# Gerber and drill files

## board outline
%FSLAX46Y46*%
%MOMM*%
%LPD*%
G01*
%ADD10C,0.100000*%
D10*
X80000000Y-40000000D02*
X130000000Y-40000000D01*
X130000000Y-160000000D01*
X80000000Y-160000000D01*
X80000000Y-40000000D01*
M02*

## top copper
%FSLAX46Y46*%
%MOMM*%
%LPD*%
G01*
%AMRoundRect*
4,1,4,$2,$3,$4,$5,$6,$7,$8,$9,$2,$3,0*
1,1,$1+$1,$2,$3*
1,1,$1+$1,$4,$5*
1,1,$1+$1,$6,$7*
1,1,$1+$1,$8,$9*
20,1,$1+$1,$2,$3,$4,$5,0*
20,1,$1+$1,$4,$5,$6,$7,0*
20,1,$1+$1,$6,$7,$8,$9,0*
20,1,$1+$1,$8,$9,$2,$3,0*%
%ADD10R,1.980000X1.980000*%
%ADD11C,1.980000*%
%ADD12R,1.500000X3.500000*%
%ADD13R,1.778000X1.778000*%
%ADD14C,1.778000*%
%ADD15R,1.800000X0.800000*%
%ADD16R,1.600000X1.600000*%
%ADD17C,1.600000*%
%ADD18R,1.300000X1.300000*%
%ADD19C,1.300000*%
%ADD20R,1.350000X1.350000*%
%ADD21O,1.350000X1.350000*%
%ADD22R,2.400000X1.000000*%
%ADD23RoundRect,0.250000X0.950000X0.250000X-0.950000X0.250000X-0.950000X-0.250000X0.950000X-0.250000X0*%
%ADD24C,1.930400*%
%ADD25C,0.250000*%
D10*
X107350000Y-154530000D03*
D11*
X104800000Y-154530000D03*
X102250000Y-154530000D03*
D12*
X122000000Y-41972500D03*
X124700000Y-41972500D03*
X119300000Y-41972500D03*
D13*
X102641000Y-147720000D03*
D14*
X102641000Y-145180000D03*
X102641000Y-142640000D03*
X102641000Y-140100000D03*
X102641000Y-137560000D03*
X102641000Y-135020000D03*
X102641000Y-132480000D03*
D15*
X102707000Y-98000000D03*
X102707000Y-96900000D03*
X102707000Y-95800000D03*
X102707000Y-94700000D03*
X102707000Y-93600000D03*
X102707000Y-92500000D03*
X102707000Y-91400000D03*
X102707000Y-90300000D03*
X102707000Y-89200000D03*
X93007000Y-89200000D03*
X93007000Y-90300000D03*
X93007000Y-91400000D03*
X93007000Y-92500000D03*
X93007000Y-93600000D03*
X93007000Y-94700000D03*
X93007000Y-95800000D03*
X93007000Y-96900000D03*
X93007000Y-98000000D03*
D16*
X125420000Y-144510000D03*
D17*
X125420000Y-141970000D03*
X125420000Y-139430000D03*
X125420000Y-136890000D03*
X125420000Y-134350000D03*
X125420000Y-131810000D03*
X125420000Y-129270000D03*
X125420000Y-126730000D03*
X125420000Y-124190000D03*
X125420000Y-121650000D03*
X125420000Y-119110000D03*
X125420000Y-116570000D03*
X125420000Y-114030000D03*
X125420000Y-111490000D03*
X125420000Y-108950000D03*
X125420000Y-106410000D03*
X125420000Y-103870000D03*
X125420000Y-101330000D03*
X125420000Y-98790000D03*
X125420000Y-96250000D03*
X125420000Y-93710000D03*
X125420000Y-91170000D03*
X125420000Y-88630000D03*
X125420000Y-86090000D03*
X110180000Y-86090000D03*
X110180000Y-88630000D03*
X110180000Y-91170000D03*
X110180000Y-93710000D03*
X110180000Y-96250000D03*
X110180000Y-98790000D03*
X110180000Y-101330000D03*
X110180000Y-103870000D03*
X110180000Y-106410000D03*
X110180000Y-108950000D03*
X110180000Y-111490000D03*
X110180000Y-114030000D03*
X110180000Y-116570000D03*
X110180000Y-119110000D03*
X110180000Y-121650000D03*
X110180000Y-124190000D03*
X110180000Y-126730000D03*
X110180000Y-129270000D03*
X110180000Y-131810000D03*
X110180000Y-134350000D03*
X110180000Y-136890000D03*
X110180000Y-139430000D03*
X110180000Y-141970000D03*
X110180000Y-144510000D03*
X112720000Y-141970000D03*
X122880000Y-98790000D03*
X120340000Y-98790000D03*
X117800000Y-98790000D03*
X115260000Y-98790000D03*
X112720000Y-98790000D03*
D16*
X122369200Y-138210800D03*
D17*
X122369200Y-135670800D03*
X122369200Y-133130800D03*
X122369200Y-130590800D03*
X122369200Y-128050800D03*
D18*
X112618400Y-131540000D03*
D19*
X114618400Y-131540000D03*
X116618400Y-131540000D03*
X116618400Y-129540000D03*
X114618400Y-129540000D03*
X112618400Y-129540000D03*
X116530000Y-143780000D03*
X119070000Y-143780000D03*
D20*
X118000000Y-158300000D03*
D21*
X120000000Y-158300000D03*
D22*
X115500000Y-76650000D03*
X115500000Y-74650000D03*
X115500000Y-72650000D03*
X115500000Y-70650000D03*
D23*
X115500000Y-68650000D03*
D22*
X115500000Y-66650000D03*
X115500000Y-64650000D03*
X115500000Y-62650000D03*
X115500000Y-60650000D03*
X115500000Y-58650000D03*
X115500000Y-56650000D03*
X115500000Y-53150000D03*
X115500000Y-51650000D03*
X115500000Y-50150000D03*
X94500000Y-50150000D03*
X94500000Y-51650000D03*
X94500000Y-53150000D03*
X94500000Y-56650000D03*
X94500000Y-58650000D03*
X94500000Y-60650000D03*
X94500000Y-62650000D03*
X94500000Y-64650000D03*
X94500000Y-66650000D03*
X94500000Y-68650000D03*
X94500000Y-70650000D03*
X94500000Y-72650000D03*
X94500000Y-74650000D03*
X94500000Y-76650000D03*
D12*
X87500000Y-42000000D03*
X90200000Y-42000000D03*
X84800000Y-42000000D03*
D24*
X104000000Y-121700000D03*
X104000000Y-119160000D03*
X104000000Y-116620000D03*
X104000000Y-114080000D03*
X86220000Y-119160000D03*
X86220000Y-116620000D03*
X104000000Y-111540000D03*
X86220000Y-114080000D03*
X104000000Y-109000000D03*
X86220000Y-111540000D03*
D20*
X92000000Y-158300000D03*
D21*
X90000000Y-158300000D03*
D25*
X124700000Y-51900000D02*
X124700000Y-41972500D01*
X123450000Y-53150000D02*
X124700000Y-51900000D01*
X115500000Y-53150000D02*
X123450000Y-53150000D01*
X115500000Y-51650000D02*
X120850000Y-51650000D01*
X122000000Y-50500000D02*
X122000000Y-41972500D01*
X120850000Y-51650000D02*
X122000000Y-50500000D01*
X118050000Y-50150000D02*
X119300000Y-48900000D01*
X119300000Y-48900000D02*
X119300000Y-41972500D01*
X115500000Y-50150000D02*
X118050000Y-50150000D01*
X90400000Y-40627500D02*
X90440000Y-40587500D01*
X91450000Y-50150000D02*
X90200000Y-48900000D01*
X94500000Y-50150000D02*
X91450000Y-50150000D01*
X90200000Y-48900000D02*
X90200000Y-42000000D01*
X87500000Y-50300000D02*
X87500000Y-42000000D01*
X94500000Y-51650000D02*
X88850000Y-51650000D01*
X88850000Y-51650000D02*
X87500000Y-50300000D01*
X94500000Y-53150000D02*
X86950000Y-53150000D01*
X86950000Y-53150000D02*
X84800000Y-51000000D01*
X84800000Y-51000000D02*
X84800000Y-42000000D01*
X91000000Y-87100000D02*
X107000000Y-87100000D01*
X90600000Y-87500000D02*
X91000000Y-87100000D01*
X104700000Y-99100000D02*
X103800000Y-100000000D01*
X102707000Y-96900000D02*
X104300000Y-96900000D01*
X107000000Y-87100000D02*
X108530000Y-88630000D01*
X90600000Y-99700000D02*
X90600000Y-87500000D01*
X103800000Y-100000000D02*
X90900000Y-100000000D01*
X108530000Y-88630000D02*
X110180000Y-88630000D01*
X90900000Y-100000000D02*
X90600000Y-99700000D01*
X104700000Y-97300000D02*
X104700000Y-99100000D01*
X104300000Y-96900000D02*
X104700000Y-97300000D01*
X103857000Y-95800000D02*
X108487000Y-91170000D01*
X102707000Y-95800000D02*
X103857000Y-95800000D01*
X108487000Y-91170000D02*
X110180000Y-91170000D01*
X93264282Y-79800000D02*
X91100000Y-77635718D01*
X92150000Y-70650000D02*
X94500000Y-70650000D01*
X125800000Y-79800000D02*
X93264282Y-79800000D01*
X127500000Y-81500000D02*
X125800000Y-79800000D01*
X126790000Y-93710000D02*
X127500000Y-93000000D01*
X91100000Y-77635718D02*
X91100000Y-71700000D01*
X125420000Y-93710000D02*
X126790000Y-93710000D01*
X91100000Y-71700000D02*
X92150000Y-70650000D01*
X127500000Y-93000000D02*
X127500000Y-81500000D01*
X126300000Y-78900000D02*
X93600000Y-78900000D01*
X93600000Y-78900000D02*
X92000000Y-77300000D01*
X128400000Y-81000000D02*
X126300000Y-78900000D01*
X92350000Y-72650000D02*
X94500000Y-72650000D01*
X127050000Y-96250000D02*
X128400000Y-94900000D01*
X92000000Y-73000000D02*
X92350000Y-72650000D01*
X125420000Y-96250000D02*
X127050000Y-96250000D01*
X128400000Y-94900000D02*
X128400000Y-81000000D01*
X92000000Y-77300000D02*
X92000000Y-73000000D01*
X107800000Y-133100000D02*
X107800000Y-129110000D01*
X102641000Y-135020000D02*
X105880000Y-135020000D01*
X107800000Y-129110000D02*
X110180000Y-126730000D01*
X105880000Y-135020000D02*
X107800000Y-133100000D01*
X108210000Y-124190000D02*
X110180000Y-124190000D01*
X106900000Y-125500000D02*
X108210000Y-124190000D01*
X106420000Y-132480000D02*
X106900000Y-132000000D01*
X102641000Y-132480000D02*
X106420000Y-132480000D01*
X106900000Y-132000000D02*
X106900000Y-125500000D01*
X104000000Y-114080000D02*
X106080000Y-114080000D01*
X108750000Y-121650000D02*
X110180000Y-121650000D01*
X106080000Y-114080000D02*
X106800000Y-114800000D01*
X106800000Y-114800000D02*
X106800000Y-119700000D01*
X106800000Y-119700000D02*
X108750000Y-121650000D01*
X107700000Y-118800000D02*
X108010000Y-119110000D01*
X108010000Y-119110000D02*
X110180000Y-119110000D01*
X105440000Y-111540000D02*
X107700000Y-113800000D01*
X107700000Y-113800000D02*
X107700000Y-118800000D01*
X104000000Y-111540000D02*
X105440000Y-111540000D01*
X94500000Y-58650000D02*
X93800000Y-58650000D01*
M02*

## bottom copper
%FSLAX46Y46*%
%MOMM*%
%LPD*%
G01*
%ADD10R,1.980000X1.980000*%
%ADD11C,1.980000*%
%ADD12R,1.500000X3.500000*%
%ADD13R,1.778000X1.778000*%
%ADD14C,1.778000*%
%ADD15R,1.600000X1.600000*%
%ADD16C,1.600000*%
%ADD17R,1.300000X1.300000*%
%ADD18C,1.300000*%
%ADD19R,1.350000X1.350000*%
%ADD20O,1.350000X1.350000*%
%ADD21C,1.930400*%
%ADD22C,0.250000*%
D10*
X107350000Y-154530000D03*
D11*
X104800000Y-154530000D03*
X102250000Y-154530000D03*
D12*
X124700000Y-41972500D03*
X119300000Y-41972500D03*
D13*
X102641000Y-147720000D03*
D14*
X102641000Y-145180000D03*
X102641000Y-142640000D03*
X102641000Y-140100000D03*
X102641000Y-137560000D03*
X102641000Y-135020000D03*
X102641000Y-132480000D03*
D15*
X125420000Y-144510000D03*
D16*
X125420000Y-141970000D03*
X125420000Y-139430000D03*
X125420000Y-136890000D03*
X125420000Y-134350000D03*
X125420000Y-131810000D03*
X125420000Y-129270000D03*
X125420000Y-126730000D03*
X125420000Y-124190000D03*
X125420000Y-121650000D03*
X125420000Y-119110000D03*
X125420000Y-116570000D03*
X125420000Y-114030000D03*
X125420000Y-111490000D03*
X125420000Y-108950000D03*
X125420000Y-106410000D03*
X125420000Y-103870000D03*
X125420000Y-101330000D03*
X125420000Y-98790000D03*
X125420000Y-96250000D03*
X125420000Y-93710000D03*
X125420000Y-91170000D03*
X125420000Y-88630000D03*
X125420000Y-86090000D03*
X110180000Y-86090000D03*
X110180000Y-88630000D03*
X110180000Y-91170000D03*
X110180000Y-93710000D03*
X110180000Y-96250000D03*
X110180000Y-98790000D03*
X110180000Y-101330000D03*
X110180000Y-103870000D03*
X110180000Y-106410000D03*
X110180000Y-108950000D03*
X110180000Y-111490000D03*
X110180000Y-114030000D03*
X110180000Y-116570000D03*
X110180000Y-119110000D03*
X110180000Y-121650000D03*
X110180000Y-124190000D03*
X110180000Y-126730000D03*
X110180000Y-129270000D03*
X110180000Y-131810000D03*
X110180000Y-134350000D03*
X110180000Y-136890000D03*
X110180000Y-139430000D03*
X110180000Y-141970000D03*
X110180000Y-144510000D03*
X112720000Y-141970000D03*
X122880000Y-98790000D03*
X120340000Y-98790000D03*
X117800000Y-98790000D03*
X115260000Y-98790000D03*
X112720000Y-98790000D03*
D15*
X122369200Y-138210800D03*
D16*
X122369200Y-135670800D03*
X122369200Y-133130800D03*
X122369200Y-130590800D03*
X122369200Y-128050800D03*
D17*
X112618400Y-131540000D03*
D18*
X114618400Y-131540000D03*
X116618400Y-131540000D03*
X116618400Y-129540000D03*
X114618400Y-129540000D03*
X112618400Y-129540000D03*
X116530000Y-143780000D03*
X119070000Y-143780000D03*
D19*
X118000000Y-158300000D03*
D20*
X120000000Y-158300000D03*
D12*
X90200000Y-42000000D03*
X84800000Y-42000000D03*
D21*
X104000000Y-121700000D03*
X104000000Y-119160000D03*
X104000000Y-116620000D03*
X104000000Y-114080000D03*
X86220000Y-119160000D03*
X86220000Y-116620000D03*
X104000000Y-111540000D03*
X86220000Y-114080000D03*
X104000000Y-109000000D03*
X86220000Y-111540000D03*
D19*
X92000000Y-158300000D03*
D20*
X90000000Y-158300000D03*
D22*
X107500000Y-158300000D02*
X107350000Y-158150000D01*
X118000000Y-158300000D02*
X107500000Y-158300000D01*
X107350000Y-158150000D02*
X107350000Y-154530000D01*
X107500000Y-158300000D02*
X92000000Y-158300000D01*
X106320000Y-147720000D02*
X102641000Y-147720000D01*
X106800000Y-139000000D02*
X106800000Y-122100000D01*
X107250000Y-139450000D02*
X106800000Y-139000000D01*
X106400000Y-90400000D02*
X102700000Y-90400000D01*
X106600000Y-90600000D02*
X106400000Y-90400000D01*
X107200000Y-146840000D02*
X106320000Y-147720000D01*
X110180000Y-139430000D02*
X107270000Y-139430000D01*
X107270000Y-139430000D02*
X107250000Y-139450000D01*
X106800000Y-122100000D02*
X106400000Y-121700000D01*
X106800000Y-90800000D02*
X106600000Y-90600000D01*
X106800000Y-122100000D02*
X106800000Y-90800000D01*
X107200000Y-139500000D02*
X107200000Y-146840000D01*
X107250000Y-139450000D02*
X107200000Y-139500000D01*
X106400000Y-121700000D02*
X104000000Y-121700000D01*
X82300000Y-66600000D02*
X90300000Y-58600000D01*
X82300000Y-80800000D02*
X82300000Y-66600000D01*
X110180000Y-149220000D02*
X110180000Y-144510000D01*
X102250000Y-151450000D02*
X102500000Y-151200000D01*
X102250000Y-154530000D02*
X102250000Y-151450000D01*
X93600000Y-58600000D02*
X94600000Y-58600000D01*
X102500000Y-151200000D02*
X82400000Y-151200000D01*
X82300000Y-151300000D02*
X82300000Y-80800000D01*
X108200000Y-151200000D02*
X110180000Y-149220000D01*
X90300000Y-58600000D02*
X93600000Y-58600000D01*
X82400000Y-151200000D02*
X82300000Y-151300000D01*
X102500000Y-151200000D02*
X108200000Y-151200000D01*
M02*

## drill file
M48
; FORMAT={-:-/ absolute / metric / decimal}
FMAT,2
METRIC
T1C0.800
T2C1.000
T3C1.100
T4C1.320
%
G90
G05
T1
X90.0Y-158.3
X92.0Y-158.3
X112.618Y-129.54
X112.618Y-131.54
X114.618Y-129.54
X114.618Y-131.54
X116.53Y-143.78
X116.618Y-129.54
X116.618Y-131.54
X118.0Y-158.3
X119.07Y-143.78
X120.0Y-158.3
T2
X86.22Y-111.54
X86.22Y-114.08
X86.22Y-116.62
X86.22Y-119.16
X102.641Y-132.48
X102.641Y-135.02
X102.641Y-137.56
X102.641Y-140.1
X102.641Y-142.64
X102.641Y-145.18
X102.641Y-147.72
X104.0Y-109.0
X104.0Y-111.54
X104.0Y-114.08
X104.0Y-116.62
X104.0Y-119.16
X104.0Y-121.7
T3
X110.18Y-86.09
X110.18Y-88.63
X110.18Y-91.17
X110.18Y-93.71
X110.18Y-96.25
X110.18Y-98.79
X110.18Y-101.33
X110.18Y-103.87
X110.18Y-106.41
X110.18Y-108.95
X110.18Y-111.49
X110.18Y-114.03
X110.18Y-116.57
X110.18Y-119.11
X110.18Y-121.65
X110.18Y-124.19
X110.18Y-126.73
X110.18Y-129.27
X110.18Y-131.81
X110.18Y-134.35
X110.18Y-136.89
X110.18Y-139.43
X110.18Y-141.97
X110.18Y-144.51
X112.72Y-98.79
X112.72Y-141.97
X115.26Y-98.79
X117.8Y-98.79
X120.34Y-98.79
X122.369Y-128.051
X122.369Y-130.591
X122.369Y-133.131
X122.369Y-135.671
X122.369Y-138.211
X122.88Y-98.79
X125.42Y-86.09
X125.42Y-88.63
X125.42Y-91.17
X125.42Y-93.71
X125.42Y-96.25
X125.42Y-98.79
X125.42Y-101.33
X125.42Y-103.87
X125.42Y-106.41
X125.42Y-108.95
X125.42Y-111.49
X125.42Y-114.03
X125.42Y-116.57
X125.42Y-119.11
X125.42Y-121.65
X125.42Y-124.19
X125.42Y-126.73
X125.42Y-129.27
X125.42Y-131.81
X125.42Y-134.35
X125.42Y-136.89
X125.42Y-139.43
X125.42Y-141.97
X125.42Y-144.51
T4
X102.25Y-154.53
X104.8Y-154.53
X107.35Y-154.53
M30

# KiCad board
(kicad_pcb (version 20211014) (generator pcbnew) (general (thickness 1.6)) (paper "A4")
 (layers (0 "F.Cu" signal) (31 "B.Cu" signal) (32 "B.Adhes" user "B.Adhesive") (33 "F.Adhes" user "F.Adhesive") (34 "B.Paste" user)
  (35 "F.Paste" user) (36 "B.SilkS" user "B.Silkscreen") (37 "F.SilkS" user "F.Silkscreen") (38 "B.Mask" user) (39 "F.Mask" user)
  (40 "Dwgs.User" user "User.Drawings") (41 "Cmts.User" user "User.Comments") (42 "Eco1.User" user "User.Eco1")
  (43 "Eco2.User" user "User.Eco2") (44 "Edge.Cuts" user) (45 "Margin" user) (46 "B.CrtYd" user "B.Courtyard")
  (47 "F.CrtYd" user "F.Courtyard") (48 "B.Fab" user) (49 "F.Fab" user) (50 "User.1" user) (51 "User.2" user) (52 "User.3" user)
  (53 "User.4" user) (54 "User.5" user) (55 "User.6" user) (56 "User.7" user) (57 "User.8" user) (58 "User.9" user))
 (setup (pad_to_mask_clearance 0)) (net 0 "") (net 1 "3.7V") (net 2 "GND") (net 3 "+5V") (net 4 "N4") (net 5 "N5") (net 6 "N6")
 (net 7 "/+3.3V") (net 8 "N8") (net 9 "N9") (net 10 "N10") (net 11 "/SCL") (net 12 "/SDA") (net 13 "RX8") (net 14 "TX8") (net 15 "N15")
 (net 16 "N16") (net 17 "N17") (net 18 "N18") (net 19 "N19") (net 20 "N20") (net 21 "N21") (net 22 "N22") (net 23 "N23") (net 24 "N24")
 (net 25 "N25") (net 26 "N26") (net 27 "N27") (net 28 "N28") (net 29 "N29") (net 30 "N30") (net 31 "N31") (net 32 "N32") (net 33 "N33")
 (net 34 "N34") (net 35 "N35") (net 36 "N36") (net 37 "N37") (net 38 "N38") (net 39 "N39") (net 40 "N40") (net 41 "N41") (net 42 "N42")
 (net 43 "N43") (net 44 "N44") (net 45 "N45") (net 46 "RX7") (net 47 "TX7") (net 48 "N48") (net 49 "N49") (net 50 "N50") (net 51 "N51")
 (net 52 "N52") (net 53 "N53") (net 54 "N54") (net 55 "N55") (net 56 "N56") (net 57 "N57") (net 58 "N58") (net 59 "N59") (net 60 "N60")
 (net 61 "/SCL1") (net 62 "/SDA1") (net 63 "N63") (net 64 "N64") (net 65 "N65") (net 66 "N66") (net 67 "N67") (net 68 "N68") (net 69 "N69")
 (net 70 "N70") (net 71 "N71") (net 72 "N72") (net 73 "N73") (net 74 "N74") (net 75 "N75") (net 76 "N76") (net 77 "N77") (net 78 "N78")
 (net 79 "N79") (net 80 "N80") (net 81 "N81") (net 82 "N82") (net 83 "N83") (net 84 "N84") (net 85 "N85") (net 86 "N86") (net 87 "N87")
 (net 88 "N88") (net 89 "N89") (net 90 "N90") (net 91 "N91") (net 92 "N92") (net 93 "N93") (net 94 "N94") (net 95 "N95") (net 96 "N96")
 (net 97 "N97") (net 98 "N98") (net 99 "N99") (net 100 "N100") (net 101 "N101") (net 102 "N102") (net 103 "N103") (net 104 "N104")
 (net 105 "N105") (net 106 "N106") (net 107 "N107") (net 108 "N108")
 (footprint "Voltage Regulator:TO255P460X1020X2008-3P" (layer "F.Cu") (at 107.35 154.53 180)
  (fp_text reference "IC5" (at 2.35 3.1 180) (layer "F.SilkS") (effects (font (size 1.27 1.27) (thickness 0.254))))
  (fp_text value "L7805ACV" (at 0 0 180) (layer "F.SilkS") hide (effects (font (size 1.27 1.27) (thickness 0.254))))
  (pad "1" thru_hole rect (at 0 0 180) (size 1.98 1.98) (drill 1.32) (layers *.Cu *.Mask) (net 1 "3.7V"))
  (pad "2" thru_hole circle (at 2.55 0 180) (size 1.98 1.98) (drill 1.32) (layers *.Cu *.Mask) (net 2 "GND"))
  (pad "3" thru_hole circle (at 5.1 0 180) (size 1.98 1.98) (drill 1.32) (layers *.Cu *.Mask) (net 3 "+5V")))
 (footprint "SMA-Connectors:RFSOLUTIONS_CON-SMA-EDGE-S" (layer "F.Cu") (at 122 41.9725 -90)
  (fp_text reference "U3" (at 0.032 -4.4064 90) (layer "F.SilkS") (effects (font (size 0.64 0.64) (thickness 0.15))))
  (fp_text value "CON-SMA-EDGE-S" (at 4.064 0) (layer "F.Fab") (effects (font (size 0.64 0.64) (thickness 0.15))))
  (pad "1" smd rect (at 0 0 270) (size 3.5 1.5) (layers "F.Cu" "F.Paste" "F.Mask") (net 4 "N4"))
  (pad "G1" smd rect (at 0 -2.7 270) (size 3.5 1.5) (layers "F.Cu" "F.Paste" "F.Mask") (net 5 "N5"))
  (pad "G2" smd rect (at 0 2.7 270) (size 3.5 1.5) (layers "F.Cu" "F.Paste" "F.Mask") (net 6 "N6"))
  (pad "G3" smd rect (at 0 -2.7 270) (size 3.5 1.5) (layers "B.Cu" "B.Paste" "B.Mask"))
  (pad "G4" smd rect (at 0 2.7 270) (size 3.5 1.5) (layers "B.Cu" "B.Paste" "B.Mask")))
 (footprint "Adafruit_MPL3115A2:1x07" (layer "F.Cu") (at 100.101 140.1 90)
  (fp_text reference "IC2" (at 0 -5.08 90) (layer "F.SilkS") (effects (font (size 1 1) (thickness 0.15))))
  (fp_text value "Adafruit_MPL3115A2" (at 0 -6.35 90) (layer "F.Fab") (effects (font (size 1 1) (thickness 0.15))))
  (pad "1" thru_hole rect (at -7.62 2.54 180) (size 1.778 1.778) (drill 1) (layers *.Cu *.Mask) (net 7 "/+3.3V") (solder_mask_margin 0.0508))
  (pad "2" thru_hole circle (at -5.08 2.54 90) (size 1.778 1.778) (drill 1) (layers *.Cu *.Mask) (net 2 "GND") (solder_mask_margin 0.0508))
  (pad "3" thru_hole circle (at -2.54 2.54 90) (size 1.778 1.778) (drill 1) (layers *.Cu *.Mask) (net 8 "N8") (solder_mask_margin 0.0508))
  (pad "4" thru_hole circle (at 0 2.54 90) (size 1.778 1.778) (drill 1) (layers *.Cu *.Mask) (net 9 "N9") (solder_mask_margin 0.0508))
  (pad "5" thru_hole circle (at 2.54 2.54 90) (size 1.778 1.778) (drill 1) (layers *.Cu *.Mask) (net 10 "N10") (solder_mask_margin 0.0508))
  (pad "6" thru_hole circle (at 5.08 2.54 90) (size 1.778 1.778) (drill 1) (layers *.Cu *.Mask) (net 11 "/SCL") (solder_mask_margin 0.0508))
  (pad "7" thru_hole circle (at 7.62 2.54 90) (size 1.778 1.778) (drill 1) (layers *.Cu *.Mask) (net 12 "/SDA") (solder_mask_margin 0.0508)))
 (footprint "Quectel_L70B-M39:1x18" (layer "F.Cu") (at 97.857 93.6 180)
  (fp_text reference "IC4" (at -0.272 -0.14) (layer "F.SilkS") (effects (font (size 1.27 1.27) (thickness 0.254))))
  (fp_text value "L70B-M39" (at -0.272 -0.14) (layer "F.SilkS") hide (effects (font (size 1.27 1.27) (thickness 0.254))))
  (pad "1" smd rect (at -4.85 -4.4 270) (size 0.8 1.8) (layers "F.Cu" "F.Paste" "F.Mask") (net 2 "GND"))
  (pad "2" smd rect (at -4.85 -3.3 270) (size 0.8 1.8) (layers "F.Cu" "F.Paste" "F.Mask") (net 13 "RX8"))
  (pad "3" smd rect (at -4.85 -2.2 270) (size 0.8 1.8) (layers "F.Cu" "F.Paste" "F.Mask") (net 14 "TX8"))
  (pad "4" smd rect (at -4.85 -1.1 270) (size 0.8 1.8) (layers "F.Cu" "F.Paste" "F.Mask") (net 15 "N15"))
  (pad "5" smd rect (at -4.85 0 270) (size 0.8 1.8) (layers "F.Cu" "F.Paste" "F.Mask") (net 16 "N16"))
  (pad "6" smd rect (at -4.85 1.1 270) (size 0.8 1.8) (layers "F.Cu" "F.Paste" "F.Mask") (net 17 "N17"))
  (pad "7" smd rect (at -4.85 2.2 270) (size 0.8 1.8) (layers "F.Cu" "F.Paste" "F.Mask") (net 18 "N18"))
  (pad "8" smd rect (at -4.85 3.3 270) (size 0.8 1.8) (layers "F.Cu" "F.Paste" "F.Mask") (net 7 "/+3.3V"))
  (pad "9" smd rect (at -4.85 4.4 270) (size 0.8 1.8) (layers "F.Cu" "F.Paste" "F.Mask") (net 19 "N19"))
  (pad "10" smd rect (at 4.85 4.4 270) (size 0.8 1.8) (layers "F.Cu" "F.Paste" "F.Mask") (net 2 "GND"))
  (pad "11" smd rect (at 4.85 3.3 270) (size 0.8 1.8) (layers "F.Cu" "F.Paste" "F.Mask") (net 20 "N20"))
  (pad "12" smd rect (at 4.85 2.2 270) (size 0.8 1.8) (layers "F.Cu" "F.Paste" "F.Mask") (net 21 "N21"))
  (pad "13" smd rect (at 4.85 1.1 270) (size 0.8 1.8) (layers "F.Cu" "F.Paste" "F.Mask") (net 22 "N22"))
  (pad "14" smd rect (at 4.85 0 270) (size 0.8 1.8) (layers "F.Cu" "F.Paste" "F.Mask") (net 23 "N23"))
  (pad "15" smd rect (at 4.85 -1.1 270) (size 0.8 1.8) (layers "F.Cu" "F.Paste" "F.Mask") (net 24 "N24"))
  (pad "16" smd rect (at 4.85 -2.2 270) (size 0.8 1.8) (layers "F.Cu" "F.Paste" "F.Mask") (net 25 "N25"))
  (pad "17" smd rect (at 4.85 -3.3 270) (size 0.8 1.8) (layers "F.Cu" "F.Paste" "F.Mask") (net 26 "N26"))
  (pad "18" smd rect (at 4.85 -4.4 270) (size 0.8 1.8) (layers "F.Cu" "F.Paste" "F.Mask") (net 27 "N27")))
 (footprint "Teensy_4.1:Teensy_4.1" (layer "F.Cu") (at 117.8 115.3 90)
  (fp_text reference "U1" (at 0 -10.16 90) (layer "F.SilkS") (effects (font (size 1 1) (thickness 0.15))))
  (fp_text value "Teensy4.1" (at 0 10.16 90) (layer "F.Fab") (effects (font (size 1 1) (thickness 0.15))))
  (pad "1" thru_hole rect (at -29.21 7.62 90) (size 1.6 1.6) (drill 1.1) (layers *.Cu *.Mask) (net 2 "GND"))
  (pad "2" thru_hole circle (at -26.67 7.62 90) (size 1.6 1.6) (drill 1.1) (layers *.Cu *.Mask) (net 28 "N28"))
  (pad "3" thru_hole circle (at -24.13 7.62 90) (size 1.6 1.6) (drill 1.1) (layers *.Cu *.Mask) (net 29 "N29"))
  (pad "4" thru_hole circle (at -21.59 7.62 90) (size 1.6 1.6) (drill 1.1) (layers *.Cu *.Mask) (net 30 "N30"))
  (pad "5" thru_hole circle (at -19.05 7.62 90) (size 1.6 1.6) (drill 1.1) (layers *.Cu *.Mask) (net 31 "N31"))
  (pad "6" thru_hole circle (at -16.51 7.62 90) (size 1.6 1.6) (drill 1.1) (layers *.Cu *.Mask) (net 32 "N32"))
  (pad "7" thru_hole circle (at -13.97 7.62 90) (size 1.6 1.6) (drill 1.1) (layers *.Cu *.Mask) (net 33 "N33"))
  (pad "8" thru_hole circle (at -11.43 7.62 90) (size 1.6 1.6) (drill 1.1) (layers *.Cu *.Mask) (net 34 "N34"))
  (pad "9" thru_hole circle (at -8.89 7.62 90) (size 1.6 1.6) (drill 1.1) (layers *.Cu *.Mask) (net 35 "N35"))
  (pad "10" thru_hole circle (at -6.35 7.62 90) (size 1.6 1.6) (drill 1.1) (layers *.Cu *.Mask) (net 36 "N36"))
  (pad "11" thru_hole circle (at -3.81 7.62 90) (size 1.6 1.6) (drill 1.1) (layers *.Cu *.Mask) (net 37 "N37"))
  (pad "12" thru_hole circle (at -1.27 7.62 90) (size 1.6 1.6) (drill 1.1) (layers *.Cu *.Mask) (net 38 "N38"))
  (pad "13" thru_hole circle (at 1.27 7.62 90) (size 1.6 1.6) (drill 1.1) (layers *.Cu *.Mask) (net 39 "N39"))
  (pad "14" thru_hole circle (at 3.81 7.62 90) (size 1.6 1.6) (drill 1.1) (layers *.Cu *.Mask) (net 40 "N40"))
  (pad "15" thru_hole circle (at 6.35 7.62 90) (size 1.6 1.6) (drill 1.1) (layers *.Cu *.Mask) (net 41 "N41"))
  (pad "16" thru_hole circle (at 8.89 7.62 90) (size 1.6 1.6) (drill 1.1) (layers *.Cu *.Mask) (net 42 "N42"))
  (pad "17" thru_hole circle (at 11.43 7.62 90) (size 1.6 1.6) (drill 1.1) (layers *.Cu *.Mask) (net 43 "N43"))
  (pad "18" thru_hole circle (at 13.97 7.62 90) (size 1.6 1.6) (drill 1.1) (layers *.Cu *.Mask) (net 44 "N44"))
  (pad "19" thru_hole circle (at 16.51 7.62 90) (size 1.6 1.6) (drill 1.1) (layers *.Cu *.Mask) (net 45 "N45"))
  (pad "20" thru_hole circle (at 19.05 7.62 90) (size 1.6 1.6) (drill 1.1) (layers *.Cu *.Mask) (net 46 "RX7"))
  (pad "21" thru_hole circle (at 21.59 7.62 90) (size 1.6 1.6) (drill 1.1) (layers *.Cu *.Mask) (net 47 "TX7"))
  (pad "22" thru_hole circle (at 24.13 7.62 90) (size 1.6 1.6) (drill 1.1) (layers *.Cu *.Mask) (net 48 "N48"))
  (pad "23" thru_hole circle (at 26.67 7.62 90) (size 1.6 1.6) (drill 1.1) (layers *.Cu *.Mask) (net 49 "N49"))
  (pad "24" thru_hole circle (at 29.21 7.62 90) (size 1.6 1.6) (drill 1.1) (layers *.Cu *.Mask) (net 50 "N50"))
  (pad "25" thru_hole circle (at 29.21 -7.62 90) (size 1.6 1.6) (drill 1.1) (layers *.Cu *.Mask) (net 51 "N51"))
  (pad "26" thru_hole circle (at 26.67 -7.62 90) (size 1.6 1.6) (drill 1.1) (layers *.Cu *.Mask) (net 13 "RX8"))
  (pad "27" thru_hole circle (at 24.13 -7.62 90) (size 1.6 1.6) (drill 1.1) (layers *.Cu *.Mask) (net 14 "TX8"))
  (pad "28" thru_hole circle (at 21.59 -7.62 90) (size 1.6 1.6) (drill 1.1) (layers *.Cu *.Mask) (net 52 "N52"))
  (pad "29" thru_hole circle (at 19.05 -7.62 90) (size 1.6 1.6) (drill 1.1) (layers *.Cu *.Mask) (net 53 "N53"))
  (pad "30" thru_hole circle (at 16.51 -7.62 90) (size 1.6 1.6) (drill 1.1) (layers *.Cu *.Mask) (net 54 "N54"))
  (pad "31" thru_hole circle (at 13.97 -7.62 90) (size 1.6 1.6) (drill 1.1) (layers *.Cu *.Mask) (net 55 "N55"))
  (pad "32" thru_hole circle (at 11.43 -7.62 90) (size 1.6 1.6) (drill 1.1) (layers *.Cu *.Mask) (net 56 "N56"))
  (pad "33" thru_hole circle (at 8.89 -7.62 90) (size 1.6 1.6) (drill 1.1) (layers *.Cu *.Mask) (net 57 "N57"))
  (pad "34" thru_hole circle (at 6.35 -7.62 90) (size 1.6 1.6) (drill 1.1) (layers *.Cu *.Mask) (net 2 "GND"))
  (pad "35" thru_hole circle (at 3.81 -7.62 90) (size 1.6 1.6) (drill 1.1) (layers *.Cu *.Mask) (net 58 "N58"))
  (pad "36" thru_hole circle (at 1.27 -7.62 90) (size 1.6 1.6) (drill 1.1) (layers *.Cu *.Mask) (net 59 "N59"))
  (pad "37" thru_hole circle (at -1.27 -7.62 90) (size 1.6 1.6) (drill 1.1) (layers *.Cu *.Mask) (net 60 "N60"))
  (pad "38" thru_hole circle (at -3.81 -7.62 90) (size 1.6 1.6) (drill 1.1) (layers *.Cu *.Mask) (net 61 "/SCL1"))
  (pad "39" thru_hole circle (at -6.35 -7.62 90) (size 1.6 1.6) (drill 1.1) (layers *.Cu *.Mask) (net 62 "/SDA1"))
  (pad "40" thru_hole circle (at -8.89 -7.62 90) (size 1.6 1.6) (drill 1.1) (layers *.Cu *.Mask) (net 12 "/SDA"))
  (pad "41" thru_hole circle (at -11.43 -7.62 90) (size 1.6 1.6) (drill 1.1) (layers *.Cu *.Mask) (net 11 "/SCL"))
  (pad "42" thru_hole circle (at -13.97 -7.62 90) (size 1.6 1.6) (drill 1.1) (layers *.Cu *.Mask) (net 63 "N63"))
  (pad "43" thru_hole circle (at -16.51 -7.62 90) (size 1.6 1.6) (drill 1.1) (layers *.Cu *.Mask) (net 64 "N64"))
  (pad "44" thru_hole circle (at -19.05 -7.62 90) (size 1.6 1.6) (drill 1.1) (layers *.Cu *.Mask) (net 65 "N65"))
  (pad "45" thru_hole circle (at -21.59 -7.62 90) (size 1.6 1.6) (drill 1.1) (layers *.Cu *.Mask) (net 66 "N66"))
  (pad "46" thru_hole circle (at -24.13 -7.62 90) (size 1.6 1.6) (drill 1.1) (layers *.Cu *.Mask) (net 7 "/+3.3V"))
  (pad "47" thru_hole circle (at -26.67 -7.62 90) (size 1.6 1.6) (drill 1.1) (layers *.Cu *.Mask) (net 2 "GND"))
  (pad "48" thru_hole circle (at -29.21 -7.62 90) (size 1.6 1.6) (drill 1.1) (layers *.Cu *.Mask) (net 3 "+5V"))
  (pad "49" thru_hole circle (at -26.67 -5.08 90) (size 1.6 1.6) (drill 1.1) (layers *.Cu *.Mask) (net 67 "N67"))
  (pad "50" thru_hole circle (at 16.51 5.08 90) (size 1.6 1.6) (drill 1.1) (layers *.Cu *.Mask) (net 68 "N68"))
  (pad "51" thru_hole circle (at 16.51 2.54 90) (size 1.6 1.6) (drill 1.1) (layers *.Cu *.Mask) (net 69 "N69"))
  (pad "52" thru_hole circle (at 16.51 0 90) (size 1.6 1.6) (drill 1.1) (layers *.Cu *.Mask) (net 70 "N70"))
  (pad "53" thru_hole circle (at 16.51 -2.54 90) (size 1.6 1.6) (drill 1.1) (layers *.Cu *.Mask) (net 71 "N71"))
  (pad "54" thru_hole circle (at 16.51 -5.08 90) (size 1.6 1.6) (drill 1.1) (layers *.Cu *.Mask) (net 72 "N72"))
  (pad "55" thru_hole rect (at -22.9108 4.5692 90) (size 1.6 1.6) (drill 1.1) (layers *.Cu *.Mask) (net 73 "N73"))
  (pad "56" thru_hole circle (at -20.3708 4.5692 90) (size 1.6 1.6) (drill 1.1) (layers *.Cu *.Mask) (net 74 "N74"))
  (pad "57" thru_hole circle (at -17.8308 4.5692 90) (size 1.6 1.6) (drill 1.1) (layers *.Cu *.Mask) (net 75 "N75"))
  (pad "58" thru_hole circle (at -15.2908 4.5692 90) (size 1.6 1.6) (drill 1.1) (layers *.Cu *.Mask) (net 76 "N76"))
  (pad "59" thru_hole circle (at -12.7508 4.5692 90) (size 1.6 1.6) (drill 1.1) (layers *.Cu *.Mask) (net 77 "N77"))
  (pad "60" thru_hole rect (at -16.24 -5.1816 90) (size 1.3 1.3) (drill 0.8) (layers *.Cu *.Mask) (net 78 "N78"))
  (pad "61" thru_hole circle (at -16.24 -3.1816 90) (size 1.3 1.3) (drill 0.8) (layers *.Cu *.Mask) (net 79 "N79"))
  (pad "62" thru_hole circle (at -16.24 -1.1816 90) (size 1.3 1.3) (drill 0.8) (layers *.Cu *.Mask) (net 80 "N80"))
  (pad "63" thru_hole circle (at -14.24 -1.1816 90) (size 1.3 1.3) (drill 0.8) (layers *.Cu *.Mask) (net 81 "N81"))
  (pad "64" thru_hole circle (at -14.24 -3.1816 90) (size 1.3 1.3) (drill 0.8) (layers *.Cu *.Mask) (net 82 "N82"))
  (pad "65" thru_hole circle (at -14.24 -5.1816 90) (size 1.3 1.3) (drill 0.8) (layers *.Cu *.Mask) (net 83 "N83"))
  (pad "66" thru_hole circle (at -28.48 -1.27 90) (size 1.3 1.3) (drill 0.8) (layers *.Cu *.Mask) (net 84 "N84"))
  (pad "67" thru_hole circle (at -28.48 1.27 90) (size 1.3 1.3) (drill 0.8) (layers *.Cu *.Mask) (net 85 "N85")))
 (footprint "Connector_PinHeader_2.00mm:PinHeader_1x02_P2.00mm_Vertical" (layer "F.Cu") (at 118 158.3 90)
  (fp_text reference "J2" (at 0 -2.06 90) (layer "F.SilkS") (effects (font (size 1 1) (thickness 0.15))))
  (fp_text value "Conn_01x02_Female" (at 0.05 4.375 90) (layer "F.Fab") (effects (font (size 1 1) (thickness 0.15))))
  (pad "1" thru_hole rect (at 0 0 90) (size 1.35 1.35) (drill 0.8) (layers *.Cu *.Mask) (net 1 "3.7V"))
  (pad "2" thru_hole oval (at 0 2 90) (size 1.35 1.35) (drill 0.8) (layers *.Cu *.Mask) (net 2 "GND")))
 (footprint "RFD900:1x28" (layer "F.Cu") (at 109.5 66.65 180)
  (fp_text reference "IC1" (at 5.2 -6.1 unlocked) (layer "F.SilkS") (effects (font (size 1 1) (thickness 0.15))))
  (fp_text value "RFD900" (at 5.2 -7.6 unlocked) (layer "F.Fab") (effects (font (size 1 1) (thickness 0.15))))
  (pad "1" smd rect (at -6 -10 180) (size 2.4 1) (layers "F.Cu" "F.Paste" "F.Mask") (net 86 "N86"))
  (pad "2" smd rect (at -6 -8 180) (size 2.4 1) (layers "F.Cu" "F.Paste" "F.Mask") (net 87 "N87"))
  (pad "3" smd rect (at -6 -6 180) (size 2.4 1) (layers "F.Cu" "F.Paste" "F.Mask") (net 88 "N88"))
  (pad "4" smd rect (at -6 -4 180) (size 2.4 1) (layers "F.Cu" "F.Paste" "F.Mask") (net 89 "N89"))
  (pad "5" smd roundrect (at -6 -2 180) (size 2.4 1) (layers "F.Cu" "F.Paste" "F.Mask") (roundrect_rratio 0.25) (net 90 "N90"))
  (pad "6" smd rect (at -6 0 180) (size 2.4 1) (layers "F.Cu" "F.Paste" "F.Mask") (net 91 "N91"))
  (pad "7" smd rect (at -6 2 180) (size 2.4 1) (layers "F.Cu" "F.Paste" "F.Mask") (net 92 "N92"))
  (pad "8" smd rect (at -6 4 180) (size 2.4 1) (layers "F.Cu" "F.Paste" "F.Mask") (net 2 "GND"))
  (pad "9" smd rect (at -6 6 180) (size 2.4 1) (layers "F.Cu" "F.Paste" "F.Mask") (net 2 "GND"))
  (pad "10" smd rect (at -6 8 180) (size 2.4 1) (layers "F.Cu" "F.Paste" "F.Mask") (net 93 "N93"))
  (pad "11" smd rect (at -6 10 180) (size 2.4 1) (layers "F.Cu" "F.Paste" "F.Mask") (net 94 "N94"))
  (pad "12" smd rect (at -6 13.5 180) (size 2.4 1) (layers "F.Cu" "F.Paste" "F.Mask") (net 5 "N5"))
  (pad "13" smd rect (at -6 15 180) (size 2.4 1) (layers "F.Cu" "F.Paste" "F.Mask") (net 4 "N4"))
  (pad "14" smd rect (at -6 16.5 180) (size 2.4 1) (layers "F.Cu" "F.Paste" "F.Mask") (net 6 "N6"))
  (pad "15" smd rect (at 15 16.5 180) (size 2.4 1) (layers "F.Cu" "F.Paste" "F.Mask") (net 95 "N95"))
  (pad "16" smd rect (at 15 15 180) (size 2.4 1) (layers "F.Cu" "F.Paste" "F.Mask") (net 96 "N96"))
  (pad "17" smd rect (at 15 13.5 180) (size 2.4 1) (layers "F.Cu" "F.Paste" "F.Mask") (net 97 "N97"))
  (pad "18" smd rect (at 15 10 180) (size 2.4 1) (layers "F.Cu" "F.Paste" "F.Mask") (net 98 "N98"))
  (pad "19" smd rect (at 15 8 180) (size 2.4 1) (layers "F.Cu" "F.Paste" "F.Mask") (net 3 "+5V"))
  (pad "20" smd rect (at 15 6 180) (size 2.4 1) (layers "F.Cu" "F.Paste" "F.Mask") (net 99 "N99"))
  (pad "21" smd rect (at 15 4 180) (size 2.4 1) (layers "F.Cu" "F.Paste" "F.Mask") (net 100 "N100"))
  (pad "22" smd rect (at 15 2 180) (size 2.4 1) (layers "F.Cu" "F.Paste" "F.Mask") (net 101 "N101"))
  (pad "23" smd rect (at 15 0 180) (size 2.4 1) (layers "F.Cu" "F.Paste" "F.Mask") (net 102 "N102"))
  (pad "24" smd rect (at 15 -2 180) (size 2.4 1) (layers "F.Cu" "F.Paste" "F.Mask") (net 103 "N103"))
  (pad "25" smd rect (at 15 -4 180) (size 2.4 1) (layers "F.Cu" "F.Paste" "F.Mask") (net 47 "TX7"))
  (pad "26" smd rect (at 15 -6 180) (size 2.4 1) (layers "F.Cu" "F.Paste" "F.Mask") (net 46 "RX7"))
  (pad "27" smd rect (at 15 -8 180) (size 2.4 1) (layers "F.Cu" "F.Paste" "F.Mask") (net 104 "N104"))
  (pad "28" smd rect (at 15 -10 180) (size 2.4 1) (layers "F.Cu" "F.Paste" "F.Mask") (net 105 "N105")))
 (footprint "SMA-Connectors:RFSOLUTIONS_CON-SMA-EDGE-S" (layer "F.Cu") (at 87.5 42 -90)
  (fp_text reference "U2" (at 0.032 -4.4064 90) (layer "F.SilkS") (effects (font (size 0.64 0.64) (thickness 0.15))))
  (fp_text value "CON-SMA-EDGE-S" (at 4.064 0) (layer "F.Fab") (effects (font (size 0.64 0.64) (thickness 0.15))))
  (pad "1" smd rect (at 0 0 270) (size 3.5 1.5) (layers "F.Cu" "F.Paste" "F.Mask") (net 96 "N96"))
  (pad "G1" smd rect (at 0 -2.7 270) (size 3.5 1.5) (layers "F.Cu" "F.Paste" "F.Mask") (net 95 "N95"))
  (pad "G2" smd rect (at 0 2.7 270) (size 3.5 1.5) (layers "F.Cu" "F.Paste" "F.Mask") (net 97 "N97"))
  (pad "G3" smd rect (at 0 -2.7 270) (size 3.5 1.5) (layers "B.Cu" "B.Paste" "B.Mask"))
  (pad "G4" smd rect (at 0 2.7 270) (size 3.5 1.5) (layers "B.Cu" "B.Paste" "B.Mask")))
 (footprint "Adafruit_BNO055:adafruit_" (layer "F.Cu") (at 104 115.35 90)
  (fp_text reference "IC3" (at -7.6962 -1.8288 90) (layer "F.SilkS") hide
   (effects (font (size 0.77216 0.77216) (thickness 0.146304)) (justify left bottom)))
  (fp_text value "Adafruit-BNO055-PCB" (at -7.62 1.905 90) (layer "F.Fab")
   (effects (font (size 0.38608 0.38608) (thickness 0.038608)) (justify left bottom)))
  (pad "1" thru_hole circle (at -6.35 0 180) (size 1.9304 1.9304) (drill 1) (layers *.Cu *.Mask) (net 7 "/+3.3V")
   (solder_mask_margin 0.0508))
  (pad "2" thru_hole circle (at -3.81 0 180) (size 1.9304 1.9304) (drill 1) (layers *.Cu *.Mask) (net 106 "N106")
   (solder_mask_margin 0.0508))
  (pad "3" thru_hole circle (at -1.27 0 180) (size 1.9304 1.9304) (drill 1) (layers *.Cu *.Mask) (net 2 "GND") (solder_mask_margin 0.0508))
  (pad "4" thru_hole circle (at 1.27 0 180) (size 1.9304 1.9304) (drill 1) (layers *.Cu *.Mask) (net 62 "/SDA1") (solder_mask_margin 0.0508))
  (pad "4" thru_hole circle (at -3.81 -17.78 180) (size 1.9304 1.9304) (drill 1) (layers *.Cu *.Mask) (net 62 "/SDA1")
   (solder_mask_margin 0.0508))
  (pad "5" thru_hole circle (at -1.27 -17.78 180) (size 1.9304 1.9304) (drill 1) (layers *.Cu *.Mask) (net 61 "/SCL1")
   (solder_mask_margin 0.0508))
  (pad "5" thru_hole circle (at 3.81 0 180) (size 1.9304 1.9304) (drill 1) (layers *.Cu *.Mask) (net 61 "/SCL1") (solder_mask_margin 0.0508))
  (pad "6" thru_hole circle (at 1.27 -17.78 180) (size 1.9304 1.9304) (drill 1) (layers *.Cu *.Mask) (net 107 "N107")
   (solder_mask_margin 0.0508))
  (pad "6" thru_hole circle (at 6.35 0 180) (size 1.9304 1.9304) (drill 1) (layers *.Cu *.Mask) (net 107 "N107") (solder_mask_margin 0.0508))
  (pad "7" thru_hole circle (at 3.81 -17.78 180) (size 1.9304 1.9304) (drill 1) (layers *.Cu *.Mask) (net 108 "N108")
   (solder_mask_margin 0.0508)))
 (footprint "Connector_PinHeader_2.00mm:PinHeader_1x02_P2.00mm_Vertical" (layer "F.Cu") (at 92 158.3 -90)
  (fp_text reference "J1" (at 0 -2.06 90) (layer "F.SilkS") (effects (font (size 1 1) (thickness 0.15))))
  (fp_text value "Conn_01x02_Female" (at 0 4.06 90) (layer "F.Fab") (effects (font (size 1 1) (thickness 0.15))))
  (pad "1" thru_hole rect (at 0 0 270) (size 1.35 1.35) (drill 0.8) (layers *.Cu *.Mask) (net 1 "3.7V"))
  (pad "2" thru_hole oval (at 0 2 270) (size 1.35 1.35) (drill 0.8) (layers *.Cu *.Mask) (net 2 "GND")))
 (gr_rect (start 130 160) (end 80 40) (layer "Edge.Cuts") (width 0.1) (fill none))
 (segment (start 124.7 51.9) (end 124.7 41.9725) (width 0.25) (layer "F.Cu") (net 5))
 (segment (start 123.45 53.15) (end 124.7 51.9) (width 0.25) (layer "F.Cu") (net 5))
 (segment (start 115.5 53.15) (end 123.45 53.15) (width 0.25) (layer "F.Cu") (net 5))
 (segment (start 115.5 51.65) (end 120.85 51.65) (width 0.25) (layer "F.Cu") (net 4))
 (segment (start 122 50.5) (end 122 41.9725) (width 0.25) (layer "F.Cu") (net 4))
 (segment (start 120.85 51.65) (end 122 50.5) (width 0.25) (layer "F.Cu") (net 4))
 (segment (start 118.05 50.15) (end 119.3 48.9) (width 0.25) (layer "F.Cu") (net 6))
 (segment (start 119.3 48.9) (end 119.3 41.9725) (width 0.25) (layer "F.Cu") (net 6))
 (segment (start 115.5 50.15) (end 118.05 50.15) (width 0.25) (layer "F.Cu") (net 6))
 (segment (start 90.4 40.6275) (end 90.44 40.5875) (width 0.25) (layer "F.Cu") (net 95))
 (segment (start 91.45 50.15) (end 90.2 48.9) (width 0.25) (layer "F.Cu") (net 95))
 (segment (start 94.5 50.15) (end 91.45 50.15) (width 0.25) (layer "F.Cu") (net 95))
 (segment (start 90.2 48.9) (end 90.2 42) (width 0.25) (layer "F.Cu") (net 95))
 (segment (start 87.5 50.3) (end 87.5 42) (width 0.25) (layer "F.Cu") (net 96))
 (segment (start 94.5 51.65) (end 88.85 51.65) (width 0.25) (layer "F.Cu") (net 96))
 (segment (start 88.85 51.65) (end 87.5 50.3) (width 0.25) (layer "F.Cu") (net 96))
 (segment (start 94.5 53.15) (end 86.95 53.15) (width 0.25) (layer "F.Cu") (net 97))
 (segment (start 86.95 53.15) (end 84.8 51) (width 0.25) (layer "F.Cu") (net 97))
 (segment (start 84.8 51) (end 84.8 42) (width 0.25) (layer "F.Cu") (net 97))
 (segment (start 107.5 158.3) (end 107.35 158.15) (width 0.25) (layer "B.Cu") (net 1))
 (segment (start 118 158.3) (end 107.5 158.3) (width 0.25) (layer "B.Cu") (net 1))
 (segment (start 107.35 158.15) (end 107.35 154.53) (width 0.25) (layer "B.Cu") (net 1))
 (segment (start 107.5 158.3) (end 92 158.3) (width 0.25) (layer "B.Cu") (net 1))
 (segment (start 91 87.1) (end 107 87.1) (width 0.25) (layer "F.Cu") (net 13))
 (segment (start 90.6 87.5) (end 91 87.1) (width 0.25) (layer "F.Cu") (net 13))
 (segment (start 104.7 99.1) (end 103.8 100) (width 0.25) (layer "F.Cu") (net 13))
 (segment (start 102.707 96.9) (end 104.3 96.9) (width 0.25) (layer "F.Cu") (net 13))
 (segment (start 107 87.1) (end 108.53 88.63) (width 0.25) (layer "F.Cu") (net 13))
 (segment (start 90.6 99.7) (end 90.6 87.5) (width 0.25) (layer "F.Cu") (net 13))
 (segment (start 103.8 100) (end 90.9 100) (width 0.25) (layer "F.Cu") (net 13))
 (segment (start 108.53 88.63) (end 110.18 88.63) (width 0.25) (layer "F.Cu") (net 13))
 (segment (start 90.9 100) (end 90.6 99.7) (width 0.25) (layer "F.Cu") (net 13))
 (segment (start 104.7 97.3) (end 104.7 99.1) (width 0.25) (layer "F.Cu") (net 13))
 (segment (start 104.3 96.9) (end 104.7 97.3) (width 0.25) (layer "F.Cu") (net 13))
 (segment (start 103.857 95.8) (end 108.487 91.17) (width 0.25) (layer "F.Cu") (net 14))
 (segment (start 102.707 95.8) (end 103.857 95.8) (width 0.25) (layer "F.Cu") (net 14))
 (segment (start 108.487 91.17) (end 110.18 91.17) (width 0.25) (layer "F.Cu") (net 14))
 (segment (start 93.264282 79.8) (end 91.1 77.635718) (width 0.25) (layer "F.Cu") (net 47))
 (segment (start 92.15 70.65) (end 94.5 70.65) (width 0.25) (layer "F.Cu") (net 47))
 (segment (start 125.8 79.8) (end 93.264282 79.8) (width 0.25) (layer "F.Cu") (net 47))
 (segment (start 127.5 81.5) (end 125.8 79.8) (width 0.25) (layer "F.Cu") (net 47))
 (segment (start 126.79 93.71) (end 127.5 93) (width 0.25) (layer "F.Cu") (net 47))
 (segment (start 91.1 77.635718) (end 91.1 71.7) (width 0.25) (layer "F.Cu") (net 47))
 (segment (start 125.42 93.71) (end 126.79 93.71) (width 0.25) (layer "F.Cu") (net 47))
 (segment (start 91.1 71.7) (end 92.15 70.65) (width 0.25) (layer "F.Cu") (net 47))
 (segment (start 127.5 93) (end 127.5 81.5) (width 0.25) (layer "F.Cu") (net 47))
 (segment (start 126.3 78.9) (end 93.6 78.9) (width 0.25) (layer "F.Cu") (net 46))
 (segment (start 93.6 78.9) (end 92 77.3) (width 0.25) (layer "F.Cu") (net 46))
 (segment (start 128.4 81) (end 126.3 78.9) (width 0.25) (layer "F.Cu") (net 46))
 (segment (start 92.35 72.65) (end 94.5 72.65) (width 0.25) (layer "F.Cu") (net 46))
 (segment (start 127.05 96.25) (end 128.4 94.9) (width 0.25) (layer "F.Cu") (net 46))
 (segment (start 92 73) (end 92.35 72.65) (width 0.25) (layer "F.Cu") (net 46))
 (segment (start 125.42 96.25) (end 127.05 96.25) (width 0.25) (layer "F.Cu") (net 46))
 (segment (start 128.4 94.9) (end 128.4 81) (width 0.25) (layer "F.Cu") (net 46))
 (segment (start 92 77.3) (end 92 73) (width 0.25) (layer "F.Cu") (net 46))
 (segment (start 106.32 147.72) (end 102.641 147.72) (width 0.25) (layer "B.Cu") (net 7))
 (segment (start 106.8 139) (end 106.8 122.1) (width 0.25) (layer "B.Cu") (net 7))
 (segment (start 107.25 139.45) (end 106.8 139) (width 0.25) (layer "B.Cu") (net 7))
 (segment (start 106.4 90.4) (end 102.7 90.4) (width 0.25) (layer "B.Cu") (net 7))
 (segment (start 106.6 90.6) (end 106.4 90.4) (width 0.25) (layer "B.Cu") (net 7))
 (segment (start 107.2 146.84) (end 106.32 147.72) (width 0.25) (layer "B.Cu") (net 7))
 (segment (start 110.18 139.43) (end 107.27 139.43) (width 0.25) (layer "B.Cu") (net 7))
 (segment (start 107.27 139.43) (end 107.25 139.45) (width 0.25) (layer "B.Cu") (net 7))
 (segment (start 106.8 122.1) (end 106.4 121.7) (width 0.25) (layer "B.Cu") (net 7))
 (segment (start 106.8 90.8) (end 106.6 90.6) (width 0.25) (layer "B.Cu") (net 7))
 (segment (start 106.8 122.1) (end 106.8 90.8) (width 0.25) (layer "B.Cu") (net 7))
 (segment (start 107.2 139.5) (end 107.2 146.84) (width 0.25) (layer "B.Cu") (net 7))
 (segment (start 107.25 139.45) (end 107.2 139.5) (width 0.25) (layer "B.Cu") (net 7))
 (segment (start 106.4 121.7) (end 104 121.7) (width 0.25) (layer "B.Cu") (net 7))
 (segment (start 107.8 133.1) (end 107.8 129.11) (width 0.25) (layer "F.Cu") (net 11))
 (segment (start 102.641 135.02) (end 105.88 135.02) (width 0.25) (layer "F.Cu") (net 11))
 (segment (start 107.8 129.11) (end 110.18 126.73) (width 0.25) (layer "F.Cu") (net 11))
 (segment (start 105.88 135.02) (end 107.8 133.1) (width 0.25) (layer "F.Cu") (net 11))
 (segment (start 108.21 124.19) (end 110.18 124.19) (width 0.25) (layer "F.Cu") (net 12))
 (segment (start 106.9 125.5) (end 108.21 124.19) (width 0.25) (layer "F.Cu") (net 12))
 (segment (start 106.42 132.48) (end 106.9 132) (width 0.25) (layer "F.Cu") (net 12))
 (segment (start 102.641 132.48) (end 106.42 132.48) (width 0.25) (layer "F.Cu") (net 12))
 (segment (start 106.9 132) (end 106.9 125.5) (width 0.25) (layer "F.Cu") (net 12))
 (segment (start 104 114.08) (end 106.08 114.08) (width 0.25) (layer "F.Cu") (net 62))
 (segment (start 108.75 121.65) (end 110.18 121.65) (width 0.25) (layer "F.Cu") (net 62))
 (segment (start 106.08 114.08) (end 106.8 114.8) (width 0.25) (layer "F.Cu") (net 62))
 (segment (start 106.8 114.8) (end 106.8 119.7) (width 0.25) (layer "F.Cu") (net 62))
 (segment (start 106.8 119.7) (end 108.75 121.65) (width 0.25) (layer "F.Cu") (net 62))
 (segment (start 107.7 118.8) (end 108.01 119.11) (width 0.25) (layer "F.Cu") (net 61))
 (segment (start 108.01 119.11) (end 110.18 119.11) (width 0.25) (layer "F.Cu") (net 61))
 (segment (start 105.44 111.54) (end 107.7 113.8) (width 0.25) (layer "F.Cu") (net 61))
 (segment (start 107.7 113.8) (end 107.7 118.8) (width 0.25) (layer "F.Cu") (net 61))
 (segment (start 104 111.54) (end 105.44 111.54) (width 0.25) (layer "F.Cu") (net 61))
 (segment (start 94.5 58.65) (end 93.8 58.65) (width 0.25) (layer "F.Cu") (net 3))
 (segment (start 82.3 66.6) (end 90.3 58.6) (width 0.25) (layer "B.Cu") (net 3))
 (segment (start 82.3 80.8) (end 82.3 66.6) (width 0.25) (layer "B.Cu") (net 3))
 (segment (start 110.18 149.22) (end 110.18 144.51) (width 0.25) (layer "B.Cu") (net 3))
 (segment (start 102.25 151.45) (end 102.5 151.2) (width 0.25) (layer "B.Cu") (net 3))
 (segment (start 102.25 154.53) (end 102.25 151.45) (width 0.25) (layer "B.Cu") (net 3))
 (segment (start 93.6 58.6) (end 94.6 58.6) (width 0.25) (layer "B.Cu") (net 3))
 (segment (start 102.5 151.2) (end 82.4 151.2) (width 0.25) (layer "B.Cu") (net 3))
 (segment (start 82.3 151.3) (end 82.3 80.8) (width 0.25) (layer "B.Cu") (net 3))
 (segment (start 108.2 151.2) (end 110.18 149.22) (width 0.25) (layer "B.Cu") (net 3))
 (segment (start 90.3 58.6) (end 93.6 58.6) (width 0.25) (layer "B.Cu") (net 3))
 (segment (start 82.4 151.2) (end 82.3 151.3) (width 0.25) (layer "B.Cu") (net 3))
 (segment (start 102.5 151.2) (end 108.2 151.2) (width 0.25) (layer "B.Cu") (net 3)))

